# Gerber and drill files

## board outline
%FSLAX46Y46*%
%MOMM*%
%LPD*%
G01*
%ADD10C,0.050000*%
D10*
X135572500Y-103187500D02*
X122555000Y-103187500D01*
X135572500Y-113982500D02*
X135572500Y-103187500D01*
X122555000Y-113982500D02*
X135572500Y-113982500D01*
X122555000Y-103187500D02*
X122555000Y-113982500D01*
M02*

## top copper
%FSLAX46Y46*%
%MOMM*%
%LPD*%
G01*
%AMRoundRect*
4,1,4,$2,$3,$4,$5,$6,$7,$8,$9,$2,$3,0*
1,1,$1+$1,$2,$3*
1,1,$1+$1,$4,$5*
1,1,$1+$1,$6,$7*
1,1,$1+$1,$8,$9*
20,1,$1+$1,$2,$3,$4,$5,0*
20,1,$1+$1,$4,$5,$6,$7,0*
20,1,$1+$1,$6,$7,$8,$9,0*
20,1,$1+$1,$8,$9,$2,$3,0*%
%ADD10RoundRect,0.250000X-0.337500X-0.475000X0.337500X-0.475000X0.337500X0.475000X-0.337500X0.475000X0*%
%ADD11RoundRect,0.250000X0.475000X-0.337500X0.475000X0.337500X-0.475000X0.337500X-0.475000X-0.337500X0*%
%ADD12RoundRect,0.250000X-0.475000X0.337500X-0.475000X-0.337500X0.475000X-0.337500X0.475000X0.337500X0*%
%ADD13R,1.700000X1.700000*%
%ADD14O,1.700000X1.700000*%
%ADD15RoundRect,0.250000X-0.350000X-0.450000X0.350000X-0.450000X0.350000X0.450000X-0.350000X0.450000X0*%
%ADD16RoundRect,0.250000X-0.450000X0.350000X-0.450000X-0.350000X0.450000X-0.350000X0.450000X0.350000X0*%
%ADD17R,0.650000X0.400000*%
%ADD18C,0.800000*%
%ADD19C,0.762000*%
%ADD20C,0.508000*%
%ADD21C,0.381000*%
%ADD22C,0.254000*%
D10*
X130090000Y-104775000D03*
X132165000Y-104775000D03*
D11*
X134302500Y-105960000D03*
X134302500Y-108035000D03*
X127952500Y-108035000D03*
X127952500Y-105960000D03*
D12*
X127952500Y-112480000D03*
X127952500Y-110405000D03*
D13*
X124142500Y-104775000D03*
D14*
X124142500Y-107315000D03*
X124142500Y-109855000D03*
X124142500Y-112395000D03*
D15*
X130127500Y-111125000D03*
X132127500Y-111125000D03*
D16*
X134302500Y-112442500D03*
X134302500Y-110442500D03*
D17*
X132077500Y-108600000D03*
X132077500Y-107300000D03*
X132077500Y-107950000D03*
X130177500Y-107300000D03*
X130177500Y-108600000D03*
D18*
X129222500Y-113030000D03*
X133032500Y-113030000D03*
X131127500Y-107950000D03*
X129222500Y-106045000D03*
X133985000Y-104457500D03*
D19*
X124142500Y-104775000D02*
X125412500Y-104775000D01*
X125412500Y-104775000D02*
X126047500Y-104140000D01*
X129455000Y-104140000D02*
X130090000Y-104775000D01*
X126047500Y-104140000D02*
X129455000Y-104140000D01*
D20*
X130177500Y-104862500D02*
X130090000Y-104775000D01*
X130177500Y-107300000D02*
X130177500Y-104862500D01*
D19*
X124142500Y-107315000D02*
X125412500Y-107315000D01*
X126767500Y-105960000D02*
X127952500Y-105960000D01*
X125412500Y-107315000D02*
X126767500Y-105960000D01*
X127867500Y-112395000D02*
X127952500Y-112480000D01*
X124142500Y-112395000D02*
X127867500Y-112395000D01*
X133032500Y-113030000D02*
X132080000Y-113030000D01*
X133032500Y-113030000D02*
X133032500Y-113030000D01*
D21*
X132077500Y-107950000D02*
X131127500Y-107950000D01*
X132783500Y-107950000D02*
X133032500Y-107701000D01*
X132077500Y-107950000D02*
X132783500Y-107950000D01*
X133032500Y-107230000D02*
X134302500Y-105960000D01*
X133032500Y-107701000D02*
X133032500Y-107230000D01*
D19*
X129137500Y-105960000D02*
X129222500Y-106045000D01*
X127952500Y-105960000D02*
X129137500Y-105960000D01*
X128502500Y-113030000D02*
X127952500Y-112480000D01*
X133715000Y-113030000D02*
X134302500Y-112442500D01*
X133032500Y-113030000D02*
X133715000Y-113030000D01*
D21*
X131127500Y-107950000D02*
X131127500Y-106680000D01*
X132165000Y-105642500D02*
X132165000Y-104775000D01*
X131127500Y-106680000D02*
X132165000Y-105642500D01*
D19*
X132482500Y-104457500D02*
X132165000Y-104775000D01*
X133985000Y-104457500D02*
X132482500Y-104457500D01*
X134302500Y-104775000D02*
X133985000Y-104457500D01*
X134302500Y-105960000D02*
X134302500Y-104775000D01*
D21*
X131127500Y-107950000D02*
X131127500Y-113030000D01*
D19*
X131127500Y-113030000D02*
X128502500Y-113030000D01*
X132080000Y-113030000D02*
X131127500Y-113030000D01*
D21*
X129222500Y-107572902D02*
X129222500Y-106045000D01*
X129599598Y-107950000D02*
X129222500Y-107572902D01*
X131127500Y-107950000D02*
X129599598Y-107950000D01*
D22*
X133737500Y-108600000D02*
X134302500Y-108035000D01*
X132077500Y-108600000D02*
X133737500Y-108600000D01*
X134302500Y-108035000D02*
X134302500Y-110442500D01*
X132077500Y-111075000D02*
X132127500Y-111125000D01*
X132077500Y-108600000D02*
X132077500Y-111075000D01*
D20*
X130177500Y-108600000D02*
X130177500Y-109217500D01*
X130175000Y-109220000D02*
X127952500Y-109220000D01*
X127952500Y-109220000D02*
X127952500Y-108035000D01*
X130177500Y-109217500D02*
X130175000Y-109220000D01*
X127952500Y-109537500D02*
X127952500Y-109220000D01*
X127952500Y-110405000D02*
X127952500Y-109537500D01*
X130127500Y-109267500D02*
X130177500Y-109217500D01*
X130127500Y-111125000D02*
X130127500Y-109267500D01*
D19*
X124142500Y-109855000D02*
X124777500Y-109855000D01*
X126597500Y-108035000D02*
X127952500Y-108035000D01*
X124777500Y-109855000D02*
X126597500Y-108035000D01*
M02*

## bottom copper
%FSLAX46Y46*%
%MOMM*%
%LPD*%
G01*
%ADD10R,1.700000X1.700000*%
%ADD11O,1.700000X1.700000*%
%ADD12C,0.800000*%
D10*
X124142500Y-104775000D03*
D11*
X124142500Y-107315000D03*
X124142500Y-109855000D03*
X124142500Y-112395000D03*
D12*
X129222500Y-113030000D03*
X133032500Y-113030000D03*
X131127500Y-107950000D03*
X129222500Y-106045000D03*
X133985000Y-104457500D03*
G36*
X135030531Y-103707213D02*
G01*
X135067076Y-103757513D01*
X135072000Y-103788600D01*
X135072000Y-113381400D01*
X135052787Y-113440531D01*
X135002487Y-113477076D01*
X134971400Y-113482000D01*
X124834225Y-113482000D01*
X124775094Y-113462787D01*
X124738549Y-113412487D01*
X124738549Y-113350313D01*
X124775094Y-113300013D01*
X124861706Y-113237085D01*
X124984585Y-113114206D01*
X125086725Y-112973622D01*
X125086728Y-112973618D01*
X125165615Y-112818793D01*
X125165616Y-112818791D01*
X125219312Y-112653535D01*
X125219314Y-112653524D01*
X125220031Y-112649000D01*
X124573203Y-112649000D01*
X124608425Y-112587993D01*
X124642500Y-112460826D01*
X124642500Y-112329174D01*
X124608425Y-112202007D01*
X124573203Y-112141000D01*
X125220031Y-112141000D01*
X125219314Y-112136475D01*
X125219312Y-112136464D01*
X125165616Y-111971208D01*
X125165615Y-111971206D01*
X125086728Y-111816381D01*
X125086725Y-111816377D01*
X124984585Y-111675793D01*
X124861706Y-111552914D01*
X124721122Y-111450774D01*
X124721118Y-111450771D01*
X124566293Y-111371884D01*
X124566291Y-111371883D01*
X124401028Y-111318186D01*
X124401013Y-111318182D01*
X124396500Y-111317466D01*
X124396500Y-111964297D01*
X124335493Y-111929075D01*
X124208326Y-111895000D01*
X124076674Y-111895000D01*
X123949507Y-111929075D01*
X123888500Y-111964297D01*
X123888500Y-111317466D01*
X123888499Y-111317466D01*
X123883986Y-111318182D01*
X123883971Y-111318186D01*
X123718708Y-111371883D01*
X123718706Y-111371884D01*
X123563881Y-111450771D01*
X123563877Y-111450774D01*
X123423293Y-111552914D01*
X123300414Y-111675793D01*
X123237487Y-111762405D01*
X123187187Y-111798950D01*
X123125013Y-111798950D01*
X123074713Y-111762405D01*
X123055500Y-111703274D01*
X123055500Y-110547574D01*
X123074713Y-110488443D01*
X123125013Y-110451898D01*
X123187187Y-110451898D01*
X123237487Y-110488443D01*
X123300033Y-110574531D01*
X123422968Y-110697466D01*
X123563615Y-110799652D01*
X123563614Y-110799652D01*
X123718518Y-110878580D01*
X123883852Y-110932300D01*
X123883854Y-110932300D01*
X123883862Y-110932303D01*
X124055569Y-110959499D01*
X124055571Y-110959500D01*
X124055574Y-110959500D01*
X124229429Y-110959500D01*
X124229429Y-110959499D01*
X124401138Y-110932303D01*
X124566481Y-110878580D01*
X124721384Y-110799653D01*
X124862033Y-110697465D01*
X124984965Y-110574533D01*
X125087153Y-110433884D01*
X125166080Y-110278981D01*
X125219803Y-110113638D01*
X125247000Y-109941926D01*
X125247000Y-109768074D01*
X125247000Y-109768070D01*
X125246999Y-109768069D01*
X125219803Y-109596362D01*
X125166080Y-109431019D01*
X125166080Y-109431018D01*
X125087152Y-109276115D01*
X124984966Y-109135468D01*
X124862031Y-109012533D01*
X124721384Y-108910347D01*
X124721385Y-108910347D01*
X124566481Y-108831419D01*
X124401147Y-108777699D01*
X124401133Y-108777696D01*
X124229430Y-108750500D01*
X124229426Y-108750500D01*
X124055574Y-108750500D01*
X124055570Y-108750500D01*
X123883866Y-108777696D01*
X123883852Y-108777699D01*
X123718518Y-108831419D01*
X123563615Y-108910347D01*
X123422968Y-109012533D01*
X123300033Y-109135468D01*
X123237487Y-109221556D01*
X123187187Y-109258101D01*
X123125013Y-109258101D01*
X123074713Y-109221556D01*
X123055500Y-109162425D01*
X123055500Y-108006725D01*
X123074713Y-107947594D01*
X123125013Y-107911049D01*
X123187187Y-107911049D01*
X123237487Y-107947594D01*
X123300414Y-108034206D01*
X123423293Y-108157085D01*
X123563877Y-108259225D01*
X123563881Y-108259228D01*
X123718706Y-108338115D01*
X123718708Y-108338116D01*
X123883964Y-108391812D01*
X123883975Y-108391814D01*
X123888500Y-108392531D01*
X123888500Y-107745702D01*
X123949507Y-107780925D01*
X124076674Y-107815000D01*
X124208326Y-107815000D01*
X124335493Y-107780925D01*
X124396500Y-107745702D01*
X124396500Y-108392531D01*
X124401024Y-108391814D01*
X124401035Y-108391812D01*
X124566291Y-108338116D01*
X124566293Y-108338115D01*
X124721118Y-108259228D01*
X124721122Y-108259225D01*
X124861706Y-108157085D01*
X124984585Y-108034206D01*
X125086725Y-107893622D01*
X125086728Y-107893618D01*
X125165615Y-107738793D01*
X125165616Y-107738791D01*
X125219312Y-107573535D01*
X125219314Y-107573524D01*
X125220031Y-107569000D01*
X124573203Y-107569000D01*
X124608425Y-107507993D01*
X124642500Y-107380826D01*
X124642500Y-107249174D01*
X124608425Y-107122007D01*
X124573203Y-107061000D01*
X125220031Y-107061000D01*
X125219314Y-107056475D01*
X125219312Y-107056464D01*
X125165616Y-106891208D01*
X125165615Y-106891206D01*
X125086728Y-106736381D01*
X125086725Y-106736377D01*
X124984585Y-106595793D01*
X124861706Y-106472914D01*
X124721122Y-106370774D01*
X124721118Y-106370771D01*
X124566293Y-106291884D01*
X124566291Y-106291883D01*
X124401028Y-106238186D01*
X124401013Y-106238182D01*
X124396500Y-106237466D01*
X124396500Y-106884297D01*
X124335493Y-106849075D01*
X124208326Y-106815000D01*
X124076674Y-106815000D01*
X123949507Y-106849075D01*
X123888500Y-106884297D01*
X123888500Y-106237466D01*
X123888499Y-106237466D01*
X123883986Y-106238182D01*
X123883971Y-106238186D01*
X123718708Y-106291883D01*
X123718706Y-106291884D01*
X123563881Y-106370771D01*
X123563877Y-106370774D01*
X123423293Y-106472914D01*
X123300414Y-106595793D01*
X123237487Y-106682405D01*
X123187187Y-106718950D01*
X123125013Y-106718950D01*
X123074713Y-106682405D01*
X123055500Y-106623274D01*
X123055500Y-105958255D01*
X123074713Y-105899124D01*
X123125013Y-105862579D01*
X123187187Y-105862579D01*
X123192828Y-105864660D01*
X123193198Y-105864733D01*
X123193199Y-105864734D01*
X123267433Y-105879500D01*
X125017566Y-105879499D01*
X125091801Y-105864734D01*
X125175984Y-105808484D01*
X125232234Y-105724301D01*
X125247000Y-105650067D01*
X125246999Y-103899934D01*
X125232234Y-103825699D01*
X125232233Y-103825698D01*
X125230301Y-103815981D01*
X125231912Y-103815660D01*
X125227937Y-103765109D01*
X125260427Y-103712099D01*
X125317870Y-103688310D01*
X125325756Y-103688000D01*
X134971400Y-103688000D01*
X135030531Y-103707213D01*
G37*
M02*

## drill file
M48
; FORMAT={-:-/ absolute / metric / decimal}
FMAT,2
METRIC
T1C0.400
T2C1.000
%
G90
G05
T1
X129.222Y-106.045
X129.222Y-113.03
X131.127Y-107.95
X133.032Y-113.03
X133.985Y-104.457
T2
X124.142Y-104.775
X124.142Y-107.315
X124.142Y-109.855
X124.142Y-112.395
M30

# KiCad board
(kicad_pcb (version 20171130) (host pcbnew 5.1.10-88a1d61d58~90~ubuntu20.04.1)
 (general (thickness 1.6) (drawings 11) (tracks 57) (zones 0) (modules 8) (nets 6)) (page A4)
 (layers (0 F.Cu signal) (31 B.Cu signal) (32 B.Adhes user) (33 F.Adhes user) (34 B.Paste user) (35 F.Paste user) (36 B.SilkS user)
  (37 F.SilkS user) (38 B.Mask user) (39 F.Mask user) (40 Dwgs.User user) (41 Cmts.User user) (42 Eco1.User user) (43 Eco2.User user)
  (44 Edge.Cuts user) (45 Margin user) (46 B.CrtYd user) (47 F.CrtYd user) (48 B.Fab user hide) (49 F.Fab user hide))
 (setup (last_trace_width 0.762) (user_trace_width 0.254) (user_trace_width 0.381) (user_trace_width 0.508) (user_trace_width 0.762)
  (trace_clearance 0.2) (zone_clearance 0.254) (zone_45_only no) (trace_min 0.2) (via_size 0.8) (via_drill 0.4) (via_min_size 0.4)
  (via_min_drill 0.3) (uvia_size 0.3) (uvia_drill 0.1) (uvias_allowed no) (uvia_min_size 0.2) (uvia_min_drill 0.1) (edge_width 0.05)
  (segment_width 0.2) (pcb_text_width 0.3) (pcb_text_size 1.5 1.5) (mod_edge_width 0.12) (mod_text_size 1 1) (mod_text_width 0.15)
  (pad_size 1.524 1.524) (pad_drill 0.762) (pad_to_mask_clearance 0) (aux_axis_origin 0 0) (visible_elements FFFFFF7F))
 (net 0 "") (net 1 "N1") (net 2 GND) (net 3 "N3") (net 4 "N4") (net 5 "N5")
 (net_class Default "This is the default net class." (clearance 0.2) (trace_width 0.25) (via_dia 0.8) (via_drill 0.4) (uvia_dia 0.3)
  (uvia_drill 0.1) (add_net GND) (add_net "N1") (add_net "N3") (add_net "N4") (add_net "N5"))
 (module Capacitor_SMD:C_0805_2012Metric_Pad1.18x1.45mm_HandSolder (layer F.Cu) (at 131.1275 104.775)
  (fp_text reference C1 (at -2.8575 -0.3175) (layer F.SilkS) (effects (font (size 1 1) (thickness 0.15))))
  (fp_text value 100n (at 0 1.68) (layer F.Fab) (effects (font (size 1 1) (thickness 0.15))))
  (pad 1 smd roundrect (at -1.0375 0) (size 1.175 1.45) (layers F.Cu F.Paste F.Mask) (roundrect_rratio 0.212766) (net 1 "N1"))
  (pad 2 smd roundrect (at 1.0375 0) (size 1.175 1.45) (layers F.Cu F.Paste F.Mask) (roundrect_rratio 0.212766) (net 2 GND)))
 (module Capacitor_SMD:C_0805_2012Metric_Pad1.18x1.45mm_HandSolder (layer F.Cu) (at 134.3025 106.9975 90)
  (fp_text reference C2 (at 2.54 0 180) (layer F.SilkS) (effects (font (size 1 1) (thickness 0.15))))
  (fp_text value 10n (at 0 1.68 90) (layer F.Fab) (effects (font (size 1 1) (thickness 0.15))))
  (pad 2 smd roundrect (at 1.0375 0 90) (size 1.175 1.45) (layers F.Cu F.Paste F.Mask) (roundrect_rratio 0.212766) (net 2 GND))
  (pad 1 smd roundrect (at -1.0375 0 90) (size 1.175 1.45) (layers F.Cu F.Paste F.Mask) (roundrect_rratio 0.212766) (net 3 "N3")))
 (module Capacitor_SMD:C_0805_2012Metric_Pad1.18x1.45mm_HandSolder (layer F.Cu) (at 127.9525 106.9975 90)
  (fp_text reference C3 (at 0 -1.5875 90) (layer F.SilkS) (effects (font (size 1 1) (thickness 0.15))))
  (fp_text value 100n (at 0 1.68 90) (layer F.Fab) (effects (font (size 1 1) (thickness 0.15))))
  (pad 1 smd roundrect (at -1.0375 0 90) (size 1.175 1.45) (layers F.Cu F.Paste F.Mask) (roundrect_rratio 0.212766) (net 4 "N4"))
  (pad 2 smd roundrect (at 1.0375 0 90) (size 1.175 1.45) (layers F.Cu F.Paste F.Mask) (roundrect_rratio 0.212766) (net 2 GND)))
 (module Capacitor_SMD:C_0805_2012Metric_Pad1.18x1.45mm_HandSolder (layer F.Cu) (at 127.9525 111.4425 270)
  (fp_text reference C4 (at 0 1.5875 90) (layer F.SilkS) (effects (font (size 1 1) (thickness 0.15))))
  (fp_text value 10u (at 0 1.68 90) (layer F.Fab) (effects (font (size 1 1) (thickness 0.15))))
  (pad 2 smd roundrect (at 1.0375 0 270) (size 1.175 1.45) (layers F.Cu F.Paste F.Mask) (roundrect_rratio 0.212766) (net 2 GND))
  (pad 1 smd roundrect (at -1.0375 0 270) (size 1.175 1.45) (layers F.Cu F.Paste F.Mask) (roundrect_rratio 0.212766) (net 4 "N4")))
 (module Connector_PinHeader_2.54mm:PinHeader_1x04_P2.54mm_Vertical (layer F.Cu) (at 124.1425 104.775)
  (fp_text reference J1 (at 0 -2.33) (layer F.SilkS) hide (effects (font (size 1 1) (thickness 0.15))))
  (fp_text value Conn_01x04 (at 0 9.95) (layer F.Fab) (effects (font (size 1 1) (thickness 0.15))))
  (pad 1 thru_hole rect (at 0 0) (size 1.7 1.7) (drill 1) (layers *.Cu *.Mask) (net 1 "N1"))
  (pad 2 thru_hole oval (at 0 2.54) (size 1.7 1.7) (drill 1) (layers *.Cu *.Mask) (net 2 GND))
  (pad 3 thru_hole oval (at 0 5.08) (size 1.7 1.7) (drill 1) (layers *.Cu *.Mask) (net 4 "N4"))
  (pad 4 thru_hole oval (at 0 7.62) (size 1.7 1.7) (drill 1) (layers *.Cu *.Mask) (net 2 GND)))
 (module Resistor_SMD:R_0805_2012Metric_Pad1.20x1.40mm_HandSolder (layer F.Cu) (at 131.1275 111.125)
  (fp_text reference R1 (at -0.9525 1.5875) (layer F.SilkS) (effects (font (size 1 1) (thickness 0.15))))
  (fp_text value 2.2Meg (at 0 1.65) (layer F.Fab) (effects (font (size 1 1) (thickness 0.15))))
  (pad 1 smd roundrect (at -1 0) (size 1.2 1.4) (layers F.Cu F.Paste F.Mask) (roundrect_rratio 0.208333) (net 4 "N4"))
  (pad 2 smd roundrect (at 1 0) (size 1.2 1.4) (layers F.Cu F.Paste F.Mask) (roundrect_rratio 0.208333) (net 3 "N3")))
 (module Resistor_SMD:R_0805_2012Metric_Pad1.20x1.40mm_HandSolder (layer F.Cu) (at 134.3025 111.4425 270)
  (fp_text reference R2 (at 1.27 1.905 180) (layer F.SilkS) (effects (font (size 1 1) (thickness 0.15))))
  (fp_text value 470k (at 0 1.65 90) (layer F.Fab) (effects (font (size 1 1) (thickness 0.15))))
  (pad 2 smd roundrect (at 1 0 270) (size 1.2 1.4) (layers F.Cu F.Paste F.Mask) (roundrect_rratio 0.208333) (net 2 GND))
  (pad 1 smd roundrect (at -1 0 270) (size 1.2 1.4) (layers F.Cu F.Paste F.Mask) (roundrect_rratio 0.208333) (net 3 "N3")))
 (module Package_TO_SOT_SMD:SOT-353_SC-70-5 (layer F.Cu) (at 131.1275 107.95 180)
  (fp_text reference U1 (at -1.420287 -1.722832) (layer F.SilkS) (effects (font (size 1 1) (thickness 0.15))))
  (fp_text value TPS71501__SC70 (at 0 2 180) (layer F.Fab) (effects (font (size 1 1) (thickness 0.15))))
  (pad 1 smd rect (at -0.95 -0.65 180) (size 0.65 0.4) (layers F.Cu F.Paste F.Mask) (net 3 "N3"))
  (pad 3 smd rect (at -0.95 0.65 180) (size 0.65 0.4) (layers F.Cu F.Paste F.Mask) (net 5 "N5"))
  (pad 2 smd rect (at -0.95 0 180) (size 0.65 0.4) (layers F.Cu F.Paste F.Mask) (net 2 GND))
  (pad 4 smd rect (at 0.95 0.65 180) (size 0.65 0.4) (layers F.Cu F.Paste F.Mask) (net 1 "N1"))
  (pad 5 smd rect (at 0.95 -0.65 180) (size 0.65 0.4) (layers F.Cu F.Paste F.Mask) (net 4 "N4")))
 (gr_line (start 135.5725 103.1875) (end 122.555 103.1875) (layer Edge.Cuts) (width 0.05))
 (gr_line (start 135.5725 113.9825) (end 135.5725 103.1875) (layer Edge.Cuts) (width 0.05))
 (gr_line (start 122.555 113.9825) (end 135.5725 113.9825) (layer Edge.Cuts) (width 0.05))
 (gr_line (start 122.555 103.1875) (end 122.555 113.9825) (layer Edge.Cuts) (width 0.05))
 (segment (start 124.1425 104.775) (end 125.4125 104.775) (width 0.762) (layer F.Cu) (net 1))
 (segment (start 125.4125 104.775) (end 126.0475 104.14) (width 0.762) (layer F.Cu) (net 1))
 (segment (start 129.455 104.14) (end 130.09 104.775) (width 0.762) (layer F.Cu) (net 1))
 (segment (start 126.0475 104.14) (end 129.455 104.14) (width 0.762) (layer F.Cu) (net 1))
 (segment (start 130.1775 104.8625) (end 130.09 104.775) (width 0.508) (layer F.Cu) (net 1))
 (segment (start 130.1775 107.3) (end 130.1775 104.8625) (width 0.508) (layer F.Cu) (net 1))
 (segment (start 124.1425 107.315) (end 125.4125 107.315) (width 0.762) (layer F.Cu) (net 2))
 (segment (start 126.7675 105.96) (end 127.9525 105.96) (width 0.762) (layer F.Cu) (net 2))
 (segment (start 125.4125 107.315) (end 126.7675 105.96) (width 0.762) (layer F.Cu) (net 2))
 (segment (start 127.8675 112.395) (end 127.9525 112.48) (width 0.762) (layer F.Cu) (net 2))
 (segment (start 124.1425 112.395) (end 127.8675 112.395) (width 0.762) (layer F.Cu) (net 2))
 (segment (start 133.0325 113.03) (end 132.08 113.03) (width 0.762) (layer F.Cu) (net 2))
 (via (at 129.2225 113.03) (size 0.8) (drill 0.4) (layers F.Cu B.Cu) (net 2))
 (segment (start 133.0325 113.03) (end 133.0325 113.03) (width 0.762) (layer F.Cu) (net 2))
 (via (at 133.0325 113.03) (size 0.8) (drill 0.4) (layers F.Cu B.Cu) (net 2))
 (via (at 131.1275 107.95) (size 0.8) (drill 0.4) (layers F.Cu B.Cu) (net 2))
 (segment (start 132.0775 107.95) (end 131.1275 107.95) (width 0.381) (layer F.Cu) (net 2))
 (segment (start 132.7835 107.95) (end 133.0325 107.701) (width 0.381) (layer F.Cu) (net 2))
 (segment (start 132.0775 107.95) (end 132.7835 107.95) (width 0.381) (layer F.Cu) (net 2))
 (segment (start 133.0325 107.23) (end 134.3025 105.96) (width 0.381) (layer F.Cu) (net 2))
 (segment (start 133.0325 107.701) (end 133.0325 107.23) (width 0.381) (layer F.Cu) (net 2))
 (via (at 129.2225 106.045) (size 0.8) (drill 0.4) (layers F.Cu B.Cu) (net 2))
 (segment (start 129.1375 105.96) (end 129.2225 106.045) (width 0.762) (layer F.Cu) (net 2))
 (segment (start 127.9525 105.96) (end 129.1375 105.96) (width 0.762) (layer F.Cu) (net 2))
 (segment (start 128.5025 113.03) (end 127.9525 112.48) (width 0.762) (layer F.Cu) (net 2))
 (segment (start 133.715 113.03) (end 134.3025 112.4425) (width 0.762) (layer F.Cu) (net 2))
 (segment (start 133.0325 113.03) (end 133.715 113.03) (width 0.762) (layer F.Cu) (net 2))
 (segment (start 131.1275 107.95) (end 131.1275 106.68) (width 0.381) (layer F.Cu) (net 2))
 (segment (start 132.165 105.6425) (end 132.165 104.775) (width 0.381) (layer F.Cu) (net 2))
 (segment (start 131.1275 106.68) (end 132.165 105.6425) (width 0.381) (layer F.Cu) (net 2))
 (via (at 133.985 104.4575) (size 0.8) (drill 0.4) (layers F.Cu B.Cu) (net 2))
 (segment (start 132.4825 104.4575) (end 132.165 104.775) (width 0.762) (layer F.Cu) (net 2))
 (segment (start 133.985 104.4575) (end 132.4825 104.4575) (width 0.762) (layer F.Cu) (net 2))
 (segment (start 134.3025 104.775) (end 133.985 104.4575) (width 0.762) (layer F.Cu) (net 2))
 (segment (start 134.3025 105.96) (end 134.3025 104.775) (width 0.762) (layer F.Cu) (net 2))
 (segment (start 131.1275 107.95) (end 131.1275 113.03) (width 0.381) (layer F.Cu) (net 2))
 (segment (start 131.1275 113.03) (end 128.5025 113.03) (width 0.762) (layer F.Cu) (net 2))
 (segment (start 132.08 113.03) (end 131.1275 113.03) (width 0.762) (layer F.Cu) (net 2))
 (segment (start 129.2225 107.572902) (end 129.2225 106.045) (width 0.381) (layer F.Cu) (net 2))
 (segment (start 129.599598 107.95) (end 129.2225 107.572902) (width 0.381) (layer F.Cu) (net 2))
 (segment (start 131.1275 107.95) (end 129.599598 107.95) (width 0.381) (layer F.Cu) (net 2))
 (segment (start 133.7375 108.6) (end 134.3025 108.035) (width 0.254) (layer F.Cu) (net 3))
 (segment (start 132.0775 108.6) (end 133.7375 108.6) (width 0.254) (layer F.Cu) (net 3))
 (segment (start 134.3025 108.035) (end 134.3025 110.4425) (width 0.254) (layer F.Cu) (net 3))
 (segment (start 132.0775 111.075) (end 132.1275 111.125) (width 0.254) (layer F.Cu) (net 3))
 (segment (start 132.0775 108.6) (end 132.0775 111.075) (width 0.254) (layer F.Cu) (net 3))
 (segment (start 130.1775 108.6) (end 130.1775 109.2175) (width 0.508) (layer F.Cu) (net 4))
 (segment (start 130.175 109.22) (end 127.9525 109.22) (width 0.508) (layer F.Cu) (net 4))
 (segment (start 127.9525 109.22) (end 127.9525 108.035) (width 0.508) (layer F.Cu) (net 4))
 (segment (start 130.1775 109.2175) (end 130.175 109.22) (width 0.508) (layer F.Cu) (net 4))
 (segment (start 127.9525 109.5375) (end 127.9525 109.22) (width 0.508) (layer F.Cu) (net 4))
 (segment (start 127.9525 110.405) (end 127.9525 109.5375) (width 0.508) (layer F.Cu) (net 4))
 (segment (start 130.1275 109.2675) (end 130.1775 109.2175) (width 0.508) (layer F.Cu) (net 4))
 (segment (start 130.1275 111.125) (end 130.1275 109.2675) (width 0.508) (layer F.Cu) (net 4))
 (segment (start 124.1425 109.855) (end 124.7775 109.855) (width 0.762) (layer F.Cu) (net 4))
 (segment (start 126.5975 108.035) (end 127.9525 108.035) (width 0.762) (layer F.Cu) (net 4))
 (segment (start 124.7775 109.855) (end 126.5975 108.035) (width 0.762) (layer F.Cu) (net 4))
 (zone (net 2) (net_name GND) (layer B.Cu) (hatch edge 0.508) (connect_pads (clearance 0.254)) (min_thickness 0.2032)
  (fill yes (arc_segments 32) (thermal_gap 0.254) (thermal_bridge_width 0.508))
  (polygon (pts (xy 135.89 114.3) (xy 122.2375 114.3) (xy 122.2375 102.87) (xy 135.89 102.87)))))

